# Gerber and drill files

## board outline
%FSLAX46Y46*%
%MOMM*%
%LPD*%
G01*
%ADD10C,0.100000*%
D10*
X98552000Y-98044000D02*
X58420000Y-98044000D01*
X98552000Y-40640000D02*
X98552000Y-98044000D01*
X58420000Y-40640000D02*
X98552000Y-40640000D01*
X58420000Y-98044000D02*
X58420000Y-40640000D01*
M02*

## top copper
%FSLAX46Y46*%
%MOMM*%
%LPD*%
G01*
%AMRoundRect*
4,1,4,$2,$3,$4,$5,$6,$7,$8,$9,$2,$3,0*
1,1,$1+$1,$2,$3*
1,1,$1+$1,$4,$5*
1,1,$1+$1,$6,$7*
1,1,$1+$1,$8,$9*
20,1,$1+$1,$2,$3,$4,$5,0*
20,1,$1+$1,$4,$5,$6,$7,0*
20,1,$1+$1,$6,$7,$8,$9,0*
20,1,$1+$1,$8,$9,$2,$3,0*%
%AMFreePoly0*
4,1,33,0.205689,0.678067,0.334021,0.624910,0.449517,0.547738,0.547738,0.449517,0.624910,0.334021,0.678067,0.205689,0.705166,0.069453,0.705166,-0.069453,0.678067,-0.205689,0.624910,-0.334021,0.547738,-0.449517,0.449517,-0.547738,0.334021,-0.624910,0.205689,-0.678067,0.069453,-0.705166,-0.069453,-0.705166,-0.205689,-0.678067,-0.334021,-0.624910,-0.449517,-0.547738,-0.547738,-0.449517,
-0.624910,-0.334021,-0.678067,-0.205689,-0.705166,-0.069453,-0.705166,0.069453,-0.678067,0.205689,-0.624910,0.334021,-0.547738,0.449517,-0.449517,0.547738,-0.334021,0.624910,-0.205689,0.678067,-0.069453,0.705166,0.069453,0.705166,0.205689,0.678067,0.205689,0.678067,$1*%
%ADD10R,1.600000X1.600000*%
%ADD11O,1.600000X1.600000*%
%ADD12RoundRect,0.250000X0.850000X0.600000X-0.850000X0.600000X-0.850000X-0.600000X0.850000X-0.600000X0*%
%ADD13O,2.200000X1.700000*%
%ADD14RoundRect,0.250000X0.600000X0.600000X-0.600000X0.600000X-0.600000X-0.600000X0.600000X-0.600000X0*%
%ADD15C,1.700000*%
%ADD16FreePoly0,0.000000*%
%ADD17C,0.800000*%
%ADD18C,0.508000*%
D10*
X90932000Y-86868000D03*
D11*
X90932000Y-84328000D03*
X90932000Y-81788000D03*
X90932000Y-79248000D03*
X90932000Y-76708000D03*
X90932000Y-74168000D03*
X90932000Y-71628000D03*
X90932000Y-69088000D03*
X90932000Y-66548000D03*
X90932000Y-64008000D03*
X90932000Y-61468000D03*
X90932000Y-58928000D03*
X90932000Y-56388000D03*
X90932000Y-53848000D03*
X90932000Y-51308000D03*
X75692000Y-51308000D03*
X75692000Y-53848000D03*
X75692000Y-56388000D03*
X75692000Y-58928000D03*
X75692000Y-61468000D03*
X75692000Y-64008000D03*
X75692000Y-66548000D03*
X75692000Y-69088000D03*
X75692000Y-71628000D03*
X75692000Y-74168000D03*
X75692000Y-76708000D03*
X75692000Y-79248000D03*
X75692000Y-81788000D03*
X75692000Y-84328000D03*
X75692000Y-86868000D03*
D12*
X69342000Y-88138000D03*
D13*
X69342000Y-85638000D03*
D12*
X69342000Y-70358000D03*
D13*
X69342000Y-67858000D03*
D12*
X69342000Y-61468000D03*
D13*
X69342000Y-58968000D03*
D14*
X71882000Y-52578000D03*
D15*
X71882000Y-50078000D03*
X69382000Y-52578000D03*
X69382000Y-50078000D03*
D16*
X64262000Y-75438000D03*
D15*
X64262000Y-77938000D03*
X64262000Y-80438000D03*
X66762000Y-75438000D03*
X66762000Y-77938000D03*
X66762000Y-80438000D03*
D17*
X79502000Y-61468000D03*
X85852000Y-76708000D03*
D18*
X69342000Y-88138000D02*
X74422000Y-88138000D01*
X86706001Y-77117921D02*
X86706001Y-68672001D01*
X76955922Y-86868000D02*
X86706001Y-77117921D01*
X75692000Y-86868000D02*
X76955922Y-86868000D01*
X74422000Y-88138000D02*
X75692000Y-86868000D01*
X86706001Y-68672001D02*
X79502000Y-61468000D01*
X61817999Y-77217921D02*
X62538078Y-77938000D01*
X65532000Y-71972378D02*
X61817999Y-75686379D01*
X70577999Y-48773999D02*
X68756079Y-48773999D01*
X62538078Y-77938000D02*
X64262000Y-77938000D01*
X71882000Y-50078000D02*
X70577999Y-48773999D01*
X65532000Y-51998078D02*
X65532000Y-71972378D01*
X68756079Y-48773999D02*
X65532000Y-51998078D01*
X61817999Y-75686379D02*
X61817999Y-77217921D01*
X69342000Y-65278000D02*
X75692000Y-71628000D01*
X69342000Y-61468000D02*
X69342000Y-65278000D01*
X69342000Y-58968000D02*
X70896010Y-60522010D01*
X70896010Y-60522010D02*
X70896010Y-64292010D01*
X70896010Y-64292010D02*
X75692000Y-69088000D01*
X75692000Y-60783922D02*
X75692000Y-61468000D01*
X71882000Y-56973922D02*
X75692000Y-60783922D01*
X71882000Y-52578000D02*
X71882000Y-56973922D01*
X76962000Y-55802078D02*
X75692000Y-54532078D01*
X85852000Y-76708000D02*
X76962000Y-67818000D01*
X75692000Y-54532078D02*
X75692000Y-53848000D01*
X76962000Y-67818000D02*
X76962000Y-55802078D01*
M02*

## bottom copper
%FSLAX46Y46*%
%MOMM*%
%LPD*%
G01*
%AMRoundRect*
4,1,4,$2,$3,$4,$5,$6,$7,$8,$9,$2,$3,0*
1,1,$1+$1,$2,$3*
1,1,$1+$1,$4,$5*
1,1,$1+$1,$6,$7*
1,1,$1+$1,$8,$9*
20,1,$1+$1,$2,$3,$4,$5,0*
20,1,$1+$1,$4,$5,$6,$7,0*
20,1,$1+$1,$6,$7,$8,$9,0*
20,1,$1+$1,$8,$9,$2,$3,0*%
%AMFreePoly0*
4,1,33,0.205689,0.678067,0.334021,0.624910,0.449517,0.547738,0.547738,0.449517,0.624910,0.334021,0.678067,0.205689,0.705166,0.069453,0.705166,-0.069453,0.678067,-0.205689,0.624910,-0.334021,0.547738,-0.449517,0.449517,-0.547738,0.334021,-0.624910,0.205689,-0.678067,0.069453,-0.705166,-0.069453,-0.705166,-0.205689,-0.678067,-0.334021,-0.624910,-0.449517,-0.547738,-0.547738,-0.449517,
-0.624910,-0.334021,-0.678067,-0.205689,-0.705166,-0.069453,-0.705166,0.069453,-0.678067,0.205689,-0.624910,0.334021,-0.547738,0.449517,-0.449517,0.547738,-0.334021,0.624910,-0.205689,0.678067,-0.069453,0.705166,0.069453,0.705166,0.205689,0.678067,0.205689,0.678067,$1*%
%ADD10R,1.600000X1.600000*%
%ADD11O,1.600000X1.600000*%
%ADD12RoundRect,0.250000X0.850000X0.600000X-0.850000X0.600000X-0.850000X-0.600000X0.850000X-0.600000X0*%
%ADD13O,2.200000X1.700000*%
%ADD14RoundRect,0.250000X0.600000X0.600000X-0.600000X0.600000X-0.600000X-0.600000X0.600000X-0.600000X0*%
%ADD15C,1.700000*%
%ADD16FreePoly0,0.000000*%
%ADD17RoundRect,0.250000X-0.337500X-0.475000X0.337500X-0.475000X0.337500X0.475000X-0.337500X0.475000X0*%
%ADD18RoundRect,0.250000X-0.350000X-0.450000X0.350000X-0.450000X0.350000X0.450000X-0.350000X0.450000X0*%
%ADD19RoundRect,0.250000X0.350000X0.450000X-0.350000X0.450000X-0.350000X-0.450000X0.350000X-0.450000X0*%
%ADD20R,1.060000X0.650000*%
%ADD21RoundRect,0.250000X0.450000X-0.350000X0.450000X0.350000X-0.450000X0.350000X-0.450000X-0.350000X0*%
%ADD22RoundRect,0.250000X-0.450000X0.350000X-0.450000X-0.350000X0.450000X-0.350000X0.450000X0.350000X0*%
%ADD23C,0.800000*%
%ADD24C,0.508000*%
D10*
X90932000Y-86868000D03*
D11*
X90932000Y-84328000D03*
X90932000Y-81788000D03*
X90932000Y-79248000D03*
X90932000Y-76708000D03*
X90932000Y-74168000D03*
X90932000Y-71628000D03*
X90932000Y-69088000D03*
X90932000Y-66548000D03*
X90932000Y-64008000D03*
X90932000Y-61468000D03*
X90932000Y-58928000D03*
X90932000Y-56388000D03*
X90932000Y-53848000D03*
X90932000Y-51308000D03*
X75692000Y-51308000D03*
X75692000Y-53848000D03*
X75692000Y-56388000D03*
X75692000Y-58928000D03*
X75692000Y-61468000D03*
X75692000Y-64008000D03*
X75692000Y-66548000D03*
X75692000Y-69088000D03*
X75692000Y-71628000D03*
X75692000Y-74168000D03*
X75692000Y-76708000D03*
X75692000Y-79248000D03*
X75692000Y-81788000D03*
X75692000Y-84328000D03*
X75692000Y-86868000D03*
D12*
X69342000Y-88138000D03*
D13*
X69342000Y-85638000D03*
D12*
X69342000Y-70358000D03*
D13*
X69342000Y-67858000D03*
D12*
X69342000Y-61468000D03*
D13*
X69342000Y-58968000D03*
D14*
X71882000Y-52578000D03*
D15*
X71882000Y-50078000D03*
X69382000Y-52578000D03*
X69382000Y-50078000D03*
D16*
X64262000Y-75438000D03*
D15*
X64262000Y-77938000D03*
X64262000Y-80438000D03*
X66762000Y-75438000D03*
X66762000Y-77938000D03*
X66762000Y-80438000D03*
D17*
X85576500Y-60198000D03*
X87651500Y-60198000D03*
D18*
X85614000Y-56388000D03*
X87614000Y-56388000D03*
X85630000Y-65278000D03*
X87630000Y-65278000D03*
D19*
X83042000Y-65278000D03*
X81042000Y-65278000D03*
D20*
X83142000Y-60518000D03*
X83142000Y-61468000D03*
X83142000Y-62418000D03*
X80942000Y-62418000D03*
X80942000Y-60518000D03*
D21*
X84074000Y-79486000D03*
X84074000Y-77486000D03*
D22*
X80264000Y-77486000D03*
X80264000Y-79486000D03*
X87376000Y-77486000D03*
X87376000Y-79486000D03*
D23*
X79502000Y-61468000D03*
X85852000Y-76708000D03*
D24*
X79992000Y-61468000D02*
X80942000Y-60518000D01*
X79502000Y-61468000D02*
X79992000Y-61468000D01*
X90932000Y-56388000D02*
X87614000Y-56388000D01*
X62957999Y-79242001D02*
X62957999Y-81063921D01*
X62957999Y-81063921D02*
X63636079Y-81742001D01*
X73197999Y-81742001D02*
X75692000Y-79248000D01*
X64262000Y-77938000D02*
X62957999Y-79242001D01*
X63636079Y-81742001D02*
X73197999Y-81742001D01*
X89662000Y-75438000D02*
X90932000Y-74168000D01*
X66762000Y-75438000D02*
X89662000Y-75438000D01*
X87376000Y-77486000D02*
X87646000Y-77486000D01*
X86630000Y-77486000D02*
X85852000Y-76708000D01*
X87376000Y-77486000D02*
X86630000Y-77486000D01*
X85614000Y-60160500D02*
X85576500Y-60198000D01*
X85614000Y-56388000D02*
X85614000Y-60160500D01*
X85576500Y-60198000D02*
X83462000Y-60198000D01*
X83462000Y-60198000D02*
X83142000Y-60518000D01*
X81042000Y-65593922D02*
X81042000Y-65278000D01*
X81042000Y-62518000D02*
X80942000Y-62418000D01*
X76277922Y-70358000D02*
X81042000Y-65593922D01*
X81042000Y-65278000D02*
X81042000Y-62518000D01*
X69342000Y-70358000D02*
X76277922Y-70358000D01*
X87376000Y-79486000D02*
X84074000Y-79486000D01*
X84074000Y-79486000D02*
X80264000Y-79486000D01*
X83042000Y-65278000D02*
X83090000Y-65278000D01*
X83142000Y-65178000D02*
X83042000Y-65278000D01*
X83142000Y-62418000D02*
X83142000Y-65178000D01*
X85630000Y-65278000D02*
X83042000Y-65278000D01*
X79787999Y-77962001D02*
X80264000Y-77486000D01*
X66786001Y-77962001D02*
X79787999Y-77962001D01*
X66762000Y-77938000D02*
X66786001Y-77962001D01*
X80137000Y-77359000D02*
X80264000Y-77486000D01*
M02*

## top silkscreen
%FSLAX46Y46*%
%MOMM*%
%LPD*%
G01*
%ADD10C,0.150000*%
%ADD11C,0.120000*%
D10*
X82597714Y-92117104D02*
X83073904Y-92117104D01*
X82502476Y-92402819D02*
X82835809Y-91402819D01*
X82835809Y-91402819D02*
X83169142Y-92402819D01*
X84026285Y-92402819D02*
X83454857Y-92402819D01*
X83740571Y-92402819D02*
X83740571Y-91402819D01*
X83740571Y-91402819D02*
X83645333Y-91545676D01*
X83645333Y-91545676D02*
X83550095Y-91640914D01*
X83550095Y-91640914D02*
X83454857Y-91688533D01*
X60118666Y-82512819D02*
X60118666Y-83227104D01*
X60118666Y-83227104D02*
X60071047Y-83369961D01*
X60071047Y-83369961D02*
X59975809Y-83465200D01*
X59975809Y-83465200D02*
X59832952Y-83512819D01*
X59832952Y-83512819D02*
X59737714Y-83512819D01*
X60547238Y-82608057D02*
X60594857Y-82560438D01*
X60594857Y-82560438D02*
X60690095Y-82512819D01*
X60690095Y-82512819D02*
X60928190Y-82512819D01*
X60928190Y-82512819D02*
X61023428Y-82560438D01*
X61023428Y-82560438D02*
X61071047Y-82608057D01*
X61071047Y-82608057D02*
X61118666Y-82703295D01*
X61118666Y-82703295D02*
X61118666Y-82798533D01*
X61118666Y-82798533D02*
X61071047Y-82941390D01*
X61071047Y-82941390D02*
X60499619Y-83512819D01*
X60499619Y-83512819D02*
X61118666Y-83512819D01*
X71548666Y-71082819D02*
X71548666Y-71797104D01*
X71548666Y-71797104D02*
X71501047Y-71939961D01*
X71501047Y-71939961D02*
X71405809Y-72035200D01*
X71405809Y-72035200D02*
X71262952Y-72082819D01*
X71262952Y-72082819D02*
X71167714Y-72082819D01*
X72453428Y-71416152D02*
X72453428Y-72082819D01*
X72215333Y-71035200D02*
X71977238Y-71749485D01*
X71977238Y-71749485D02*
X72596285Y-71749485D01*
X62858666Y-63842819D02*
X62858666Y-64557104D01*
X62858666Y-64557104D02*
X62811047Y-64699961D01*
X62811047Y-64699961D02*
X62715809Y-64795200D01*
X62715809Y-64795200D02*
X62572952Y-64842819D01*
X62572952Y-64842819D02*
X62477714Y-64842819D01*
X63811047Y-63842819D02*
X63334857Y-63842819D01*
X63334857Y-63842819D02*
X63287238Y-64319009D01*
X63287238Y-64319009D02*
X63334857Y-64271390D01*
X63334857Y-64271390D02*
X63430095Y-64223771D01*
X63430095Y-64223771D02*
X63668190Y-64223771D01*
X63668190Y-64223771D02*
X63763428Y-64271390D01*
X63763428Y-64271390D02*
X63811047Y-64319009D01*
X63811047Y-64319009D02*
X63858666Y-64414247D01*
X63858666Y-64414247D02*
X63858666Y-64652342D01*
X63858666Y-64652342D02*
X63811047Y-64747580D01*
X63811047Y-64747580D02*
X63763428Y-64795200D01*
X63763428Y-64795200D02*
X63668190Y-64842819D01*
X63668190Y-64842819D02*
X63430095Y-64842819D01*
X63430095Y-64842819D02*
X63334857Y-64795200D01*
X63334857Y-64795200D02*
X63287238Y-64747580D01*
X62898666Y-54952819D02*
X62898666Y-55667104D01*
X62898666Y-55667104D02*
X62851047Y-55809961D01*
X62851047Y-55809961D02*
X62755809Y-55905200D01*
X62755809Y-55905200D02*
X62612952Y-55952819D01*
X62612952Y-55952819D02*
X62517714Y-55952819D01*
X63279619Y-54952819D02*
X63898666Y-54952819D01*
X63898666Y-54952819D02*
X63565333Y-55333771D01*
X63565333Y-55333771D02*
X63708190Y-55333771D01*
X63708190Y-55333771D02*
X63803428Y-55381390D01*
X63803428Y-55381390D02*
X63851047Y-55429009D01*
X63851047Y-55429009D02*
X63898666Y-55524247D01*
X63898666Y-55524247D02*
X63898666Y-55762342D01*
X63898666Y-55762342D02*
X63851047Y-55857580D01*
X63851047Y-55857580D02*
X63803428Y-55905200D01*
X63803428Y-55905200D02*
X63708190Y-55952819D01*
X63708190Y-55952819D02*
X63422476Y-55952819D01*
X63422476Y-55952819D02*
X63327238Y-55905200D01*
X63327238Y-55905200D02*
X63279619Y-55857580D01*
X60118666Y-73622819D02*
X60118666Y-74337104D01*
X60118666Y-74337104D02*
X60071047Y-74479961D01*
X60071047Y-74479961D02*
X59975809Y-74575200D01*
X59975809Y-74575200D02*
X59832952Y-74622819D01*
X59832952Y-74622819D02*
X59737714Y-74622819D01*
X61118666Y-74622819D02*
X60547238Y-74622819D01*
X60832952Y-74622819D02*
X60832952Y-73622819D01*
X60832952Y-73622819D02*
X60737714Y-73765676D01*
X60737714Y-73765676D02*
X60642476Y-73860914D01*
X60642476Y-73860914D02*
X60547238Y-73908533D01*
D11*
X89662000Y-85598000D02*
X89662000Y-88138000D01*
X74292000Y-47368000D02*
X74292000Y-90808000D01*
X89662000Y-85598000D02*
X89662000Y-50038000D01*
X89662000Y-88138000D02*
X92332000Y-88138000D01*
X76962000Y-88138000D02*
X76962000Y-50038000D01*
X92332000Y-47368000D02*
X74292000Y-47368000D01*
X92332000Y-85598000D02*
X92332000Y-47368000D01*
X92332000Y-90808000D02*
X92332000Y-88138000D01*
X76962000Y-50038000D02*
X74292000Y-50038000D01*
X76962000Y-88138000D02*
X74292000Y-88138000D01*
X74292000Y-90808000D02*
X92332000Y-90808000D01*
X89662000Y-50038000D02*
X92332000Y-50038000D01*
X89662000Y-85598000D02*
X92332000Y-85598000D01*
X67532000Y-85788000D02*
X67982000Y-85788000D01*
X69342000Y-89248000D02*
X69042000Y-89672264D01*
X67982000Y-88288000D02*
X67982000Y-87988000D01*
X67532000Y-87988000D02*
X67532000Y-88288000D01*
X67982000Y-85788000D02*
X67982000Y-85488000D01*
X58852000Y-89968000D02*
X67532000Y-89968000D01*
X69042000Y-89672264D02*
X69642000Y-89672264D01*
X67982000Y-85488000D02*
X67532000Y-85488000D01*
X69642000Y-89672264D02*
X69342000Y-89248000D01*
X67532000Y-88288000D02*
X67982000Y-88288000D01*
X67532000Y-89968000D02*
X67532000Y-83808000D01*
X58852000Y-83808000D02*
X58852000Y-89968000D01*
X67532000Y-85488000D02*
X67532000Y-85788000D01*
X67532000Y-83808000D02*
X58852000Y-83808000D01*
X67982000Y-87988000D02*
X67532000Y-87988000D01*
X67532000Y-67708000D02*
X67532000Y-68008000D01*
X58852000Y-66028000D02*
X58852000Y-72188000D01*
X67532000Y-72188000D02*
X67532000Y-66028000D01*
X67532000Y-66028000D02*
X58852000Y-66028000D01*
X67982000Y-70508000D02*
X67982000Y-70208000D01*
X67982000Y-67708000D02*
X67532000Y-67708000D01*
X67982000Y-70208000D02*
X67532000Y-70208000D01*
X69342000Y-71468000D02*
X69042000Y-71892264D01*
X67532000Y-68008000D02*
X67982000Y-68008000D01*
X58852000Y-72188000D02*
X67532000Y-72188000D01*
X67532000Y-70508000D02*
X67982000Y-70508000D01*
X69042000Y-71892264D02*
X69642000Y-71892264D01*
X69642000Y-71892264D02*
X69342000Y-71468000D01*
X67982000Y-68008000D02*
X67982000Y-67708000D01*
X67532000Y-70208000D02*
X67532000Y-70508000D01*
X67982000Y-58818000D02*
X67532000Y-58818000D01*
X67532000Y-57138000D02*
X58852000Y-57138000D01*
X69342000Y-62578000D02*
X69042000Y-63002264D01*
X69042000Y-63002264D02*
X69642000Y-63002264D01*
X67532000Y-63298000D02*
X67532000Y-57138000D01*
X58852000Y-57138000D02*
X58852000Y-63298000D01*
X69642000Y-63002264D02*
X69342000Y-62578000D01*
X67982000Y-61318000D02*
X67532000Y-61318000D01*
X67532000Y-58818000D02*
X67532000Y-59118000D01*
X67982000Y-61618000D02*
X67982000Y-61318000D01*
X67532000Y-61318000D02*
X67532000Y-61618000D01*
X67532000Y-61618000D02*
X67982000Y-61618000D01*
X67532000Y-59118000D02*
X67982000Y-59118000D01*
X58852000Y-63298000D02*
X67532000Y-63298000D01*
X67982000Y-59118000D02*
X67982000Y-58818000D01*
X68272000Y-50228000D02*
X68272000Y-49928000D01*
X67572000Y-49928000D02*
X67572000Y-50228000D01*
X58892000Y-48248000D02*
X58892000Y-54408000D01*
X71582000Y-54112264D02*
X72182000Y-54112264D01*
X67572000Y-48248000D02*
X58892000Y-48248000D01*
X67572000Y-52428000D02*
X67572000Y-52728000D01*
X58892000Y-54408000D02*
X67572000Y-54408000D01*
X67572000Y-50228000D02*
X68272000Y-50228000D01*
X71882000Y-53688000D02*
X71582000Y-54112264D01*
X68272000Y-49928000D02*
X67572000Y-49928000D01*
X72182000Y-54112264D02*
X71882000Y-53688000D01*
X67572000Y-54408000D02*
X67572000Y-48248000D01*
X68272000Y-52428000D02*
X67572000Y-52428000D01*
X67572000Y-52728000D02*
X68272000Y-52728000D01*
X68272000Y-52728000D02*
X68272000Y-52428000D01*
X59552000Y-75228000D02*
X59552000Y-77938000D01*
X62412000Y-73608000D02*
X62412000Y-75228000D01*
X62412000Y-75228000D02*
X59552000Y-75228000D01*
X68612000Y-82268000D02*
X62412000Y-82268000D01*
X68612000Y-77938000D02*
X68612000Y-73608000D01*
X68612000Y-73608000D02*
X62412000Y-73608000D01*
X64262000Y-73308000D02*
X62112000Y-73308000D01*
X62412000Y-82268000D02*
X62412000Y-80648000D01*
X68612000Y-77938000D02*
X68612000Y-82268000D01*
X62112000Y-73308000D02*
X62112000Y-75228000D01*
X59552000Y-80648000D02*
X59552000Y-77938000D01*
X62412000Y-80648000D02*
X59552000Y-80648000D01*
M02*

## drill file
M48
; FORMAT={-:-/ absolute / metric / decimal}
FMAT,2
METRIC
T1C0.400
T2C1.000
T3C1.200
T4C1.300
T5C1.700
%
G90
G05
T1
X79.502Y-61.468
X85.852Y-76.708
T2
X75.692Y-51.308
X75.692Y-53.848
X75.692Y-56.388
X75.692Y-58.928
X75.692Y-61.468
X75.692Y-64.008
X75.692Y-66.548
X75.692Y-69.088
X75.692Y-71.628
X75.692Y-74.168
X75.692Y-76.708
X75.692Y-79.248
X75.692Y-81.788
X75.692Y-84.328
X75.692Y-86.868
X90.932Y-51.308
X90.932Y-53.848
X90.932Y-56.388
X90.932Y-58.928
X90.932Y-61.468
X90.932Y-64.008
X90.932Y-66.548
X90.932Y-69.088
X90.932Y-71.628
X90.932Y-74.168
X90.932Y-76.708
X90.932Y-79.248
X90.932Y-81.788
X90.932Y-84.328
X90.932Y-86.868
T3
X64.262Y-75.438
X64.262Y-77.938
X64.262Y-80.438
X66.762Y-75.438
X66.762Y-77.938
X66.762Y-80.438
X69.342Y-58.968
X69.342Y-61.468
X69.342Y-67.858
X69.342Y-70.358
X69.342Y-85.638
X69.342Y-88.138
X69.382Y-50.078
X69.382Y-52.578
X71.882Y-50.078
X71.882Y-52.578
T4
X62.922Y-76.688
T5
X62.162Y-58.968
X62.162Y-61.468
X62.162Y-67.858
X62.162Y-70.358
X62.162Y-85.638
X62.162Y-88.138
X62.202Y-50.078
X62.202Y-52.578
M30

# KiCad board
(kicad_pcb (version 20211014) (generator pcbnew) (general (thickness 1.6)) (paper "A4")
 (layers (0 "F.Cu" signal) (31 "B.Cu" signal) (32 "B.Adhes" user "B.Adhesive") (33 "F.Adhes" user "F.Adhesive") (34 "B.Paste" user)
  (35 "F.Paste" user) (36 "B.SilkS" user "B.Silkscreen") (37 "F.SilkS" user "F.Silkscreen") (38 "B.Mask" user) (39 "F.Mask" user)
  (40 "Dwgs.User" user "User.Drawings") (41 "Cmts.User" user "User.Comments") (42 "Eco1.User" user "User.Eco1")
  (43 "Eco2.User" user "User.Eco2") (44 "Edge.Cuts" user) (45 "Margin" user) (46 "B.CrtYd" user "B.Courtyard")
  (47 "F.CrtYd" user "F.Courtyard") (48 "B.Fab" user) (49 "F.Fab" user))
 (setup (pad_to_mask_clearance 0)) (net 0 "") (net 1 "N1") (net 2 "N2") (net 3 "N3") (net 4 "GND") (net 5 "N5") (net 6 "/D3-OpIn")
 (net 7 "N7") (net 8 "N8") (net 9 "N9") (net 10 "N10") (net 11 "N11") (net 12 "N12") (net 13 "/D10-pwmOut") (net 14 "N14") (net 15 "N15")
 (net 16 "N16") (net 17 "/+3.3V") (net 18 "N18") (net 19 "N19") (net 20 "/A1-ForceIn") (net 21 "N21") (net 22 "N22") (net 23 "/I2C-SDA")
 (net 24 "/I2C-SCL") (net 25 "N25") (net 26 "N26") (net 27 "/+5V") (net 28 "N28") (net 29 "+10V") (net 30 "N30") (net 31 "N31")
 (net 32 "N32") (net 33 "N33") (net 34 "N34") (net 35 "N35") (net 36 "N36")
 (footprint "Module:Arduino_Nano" (layer "F.Cu") (at 90.932 86.868 180)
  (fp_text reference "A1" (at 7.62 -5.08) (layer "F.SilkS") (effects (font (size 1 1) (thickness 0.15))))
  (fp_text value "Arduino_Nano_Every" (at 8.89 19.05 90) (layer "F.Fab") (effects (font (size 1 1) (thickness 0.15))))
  (fp_line (start 1.27 1.27) (end 1.27 -1.27) (layer "F.SilkS") (width 0.12))
  (fp_line (start 16.64 39.5) (end 16.64 -3.94) (layer "F.SilkS") (width 0.12))
  (fp_line (start 1.27 1.27) (end 1.27 36.83) (layer "F.SilkS") (width 0.12))
  (fp_line (start 1.27 -1.27) (end -1.4 -1.27) (layer "F.SilkS") (width 0.12))
  (fp_line (start 13.97 -1.27) (end 13.97 36.83) (layer "F.SilkS") (width 0.12))
  (fp_line (start -1.4 39.5) (end 16.64 39.5) (layer "F.SilkS") (width 0.12))
  (fp_line (start -1.4 1.27) (end -1.4 39.5) (layer "F.SilkS") (width 0.12))
  (fp_line (start -1.4 -3.94) (end -1.4 -1.27) (layer "F.SilkS") (width 0.12))
  (fp_line (start 13.97 36.83) (end 16.64 36.83) (layer "F.SilkS") (width 0.12))
  (fp_line (start 13.97 -1.27) (end 16.64 -1.27) (layer "F.SilkS") (width 0.12))
  (fp_line (start 16.64 -3.94) (end -1.4 -3.94) (layer "F.SilkS") (width 0.12))
  (fp_line (start 1.27 36.83) (end -1.4 36.83) (layer "F.SilkS") (width 0.12))
  (fp_line (start 1.27 1.27) (end -1.4 1.27) (layer "F.SilkS") (width 0.12))
  (pad "1" thru_hole rect locked (at 0 0 180) (size 1.6 1.6) (drill 1) (layers *.Cu *.Mask) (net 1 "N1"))
  (pad "2" thru_hole oval locked (at 0 2.54 180) (size 1.6 1.6) (drill 1) (layers *.Cu *.Mask) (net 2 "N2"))
  (pad "3" thru_hole oval locked (at 0 5.08 180) (size 1.6 1.6) (drill 1) (layers *.Cu *.Mask) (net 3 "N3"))
  (pad "4" thru_hole oval locked (at 0 7.62 180) (size 1.6 1.6) (drill 1) (layers *.Cu *.Mask) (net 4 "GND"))
  (pad "5" thru_hole oval locked (at 0 10.16 180) (size 1.6 1.6) (drill 1) (layers *.Cu *.Mask) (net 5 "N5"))
  (pad "6" thru_hole oval locked (at 0 12.7 180) (size 1.6 1.6) (drill 1) (layers *.Cu *.Mask) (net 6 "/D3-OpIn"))
  (pad "7" thru_hole oval locked (at 0 15.24 180) (size 1.6 1.6) (drill 1) (layers *.Cu *.Mask) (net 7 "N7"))
  (pad "8" thru_hole oval locked (at 0 17.78 180) (size 1.6 1.6) (drill 1) (layers *.Cu *.Mask) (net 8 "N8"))
  (pad "9" thru_hole oval locked (at 0 20.32 180) (size 1.6 1.6) (drill 1) (layers *.Cu *.Mask) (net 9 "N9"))
  (pad "10" thru_hole oval locked (at 0 22.86 180) (size 1.6 1.6) (drill 1) (layers *.Cu *.Mask) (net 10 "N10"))
  (pad "11" thru_hole oval locked (at 0 25.4 180) (size 1.6 1.6) (drill 1) (layers *.Cu *.Mask) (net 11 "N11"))
  (pad "12" thru_hole oval locked (at 0 27.94 180) (size 1.6 1.6) (drill 1) (layers *.Cu *.Mask) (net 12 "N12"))
  (pad "13" thru_hole oval locked (at 0 30.48 180) (size 1.6 1.6) (drill 1) (layers *.Cu *.Mask) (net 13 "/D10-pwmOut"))
  (pad "14" thru_hole oval locked (at 0 33.02 180) (size 1.6 1.6) (drill 1) (layers *.Cu *.Mask) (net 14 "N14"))
  (pad "15" thru_hole oval locked (at 0 35.56 180) (size 1.6 1.6) (drill 1) (layers *.Cu *.Mask) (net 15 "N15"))
  (pad "16" thru_hole oval locked (at 15.24 35.56 180) (size 1.6 1.6) (drill 1) (layers *.Cu *.Mask) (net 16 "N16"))
  (pad "17" thru_hole oval locked (at 15.24 33.02 180) (size 1.6 1.6) (drill 1) (layers *.Cu *.Mask) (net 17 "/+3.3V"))
  (pad "18" thru_hole oval locked (at 15.24 30.48 180) (size 1.6 1.6) (drill 1) (layers *.Cu *.Mask) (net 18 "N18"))
  (pad "19" thru_hole oval locked (at 15.24 27.94 180) (size 1.6 1.6) (drill 1) (layers *.Cu *.Mask) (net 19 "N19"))
  (pad "20" thru_hole oval locked (at 15.24 25.4 180) (size 1.6 1.6) (drill 1) (layers *.Cu *.Mask) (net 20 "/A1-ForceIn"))
  (pad "21" thru_hole oval locked (at 15.24 22.86 180) (size 1.6 1.6) (drill 1) (layers *.Cu *.Mask) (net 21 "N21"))
  (pad "22" thru_hole oval locked (at 15.24 20.32 180) (size 1.6 1.6) (drill 1) (layers *.Cu *.Mask) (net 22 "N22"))
  (pad "23" thru_hole oval locked (at 15.24 17.78 180) (size 1.6 1.6) (drill 1) (layers *.Cu *.Mask) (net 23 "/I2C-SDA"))
  (pad "24" thru_hole oval locked (at 15.24 15.24 180) (size 1.6 1.6) (drill 1) (layers *.Cu *.Mask) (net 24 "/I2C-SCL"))
  (pad "25" thru_hole oval locked (at 15.24 12.7 180) (size 1.6 1.6) (drill 1) (layers *.Cu *.Mask) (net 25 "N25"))
  (pad "26" thru_hole oval locked (at 15.24 10.16 180) (size 1.6 1.6) (drill 1) (layers *.Cu *.Mask) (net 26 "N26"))
  (pad "27" thru_hole oval locked (at 15.24 7.62 180) (size 1.6 1.6) (drill 1) (layers *.Cu *.Mask) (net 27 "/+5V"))
  (pad "28" thru_hole oval locked (at 15.24 5.08 180) (size 1.6 1.6) (drill 1) (layers *.Cu *.Mask) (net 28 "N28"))
  (pad "29" thru_hole oval locked (at 15.24 2.54 180) (size 1.6 1.6) (drill 1) (layers *.Cu *.Mask) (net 4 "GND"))
  (pad "30" thru_hole oval locked (at 15.24 0 180) (size 1.6 1.6) (drill 1) (layers *.Cu *.Mask) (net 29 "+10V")))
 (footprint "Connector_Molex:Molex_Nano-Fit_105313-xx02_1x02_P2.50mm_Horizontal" (layer "F.Cu") (at 69.342 88.138 180)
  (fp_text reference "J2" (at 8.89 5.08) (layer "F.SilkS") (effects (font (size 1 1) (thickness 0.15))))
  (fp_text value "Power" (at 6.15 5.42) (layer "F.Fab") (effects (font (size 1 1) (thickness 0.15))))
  (fp_line (start 1.81 2.35) (end 1.36 2.35) (layer "F.SilkS") (width 0.12))
  (fp_line (start 0 -1.11) (end 0.3 -1.534264) (layer "F.SilkS") (width 0.12))
  (fp_line (start 1.36 -0.15) (end 1.36 0.15) (layer "F.SilkS") (width 0.12))
  (fp_line (start 1.81 0.15) (end 1.81 -0.15) (layer "F.SilkS") (width 0.12))
  (fp_line (start 1.36 2.35) (end 1.36 2.65) (layer "F.SilkS") (width 0.12))
  (fp_line (start 10.49 -1.83) (end 1.81 -1.83) (layer "F.SilkS") (width 0.12))
  (fp_line (start 0.3 -1.534264) (end -0.3 -1.534264) (layer "F.SilkS") (width 0.12))
  (fp_line (start 1.36 2.65) (end 1.81 2.65) (layer "F.SilkS") (width 0.12))
  (fp_line (start -0.3 -1.534264) (end 0 -1.11) (layer "F.SilkS") (width 0.12))
  (fp_line (start 1.81 -0.15) (end 1.36 -0.15) (layer "F.SilkS") (width 0.12))
  (fp_line (start 1.81 -1.83) (end 1.81 4.33) (layer "F.SilkS") (width 0.12))
  (fp_line (start 10.49 4.33) (end 10.49 -1.83) (layer "F.SilkS") (width 0.12))
  (fp_line (start 1.81 2.65) (end 1.81 2.35) (layer "F.SilkS") (width 0.12))
  (fp_line (start 1.81 4.33) (end 10.49 4.33) (layer "F.SilkS") (width 0.12))
  (fp_line (start 1.36 0.15) (end 1.81 0.15) (layer "F.SilkS") (width 0.12))
  (pad "" np_thru_hole circle locked (at 7.18 2.5 180) (size 1.7 1.7) (drill 1.7) (layers *.Cu *.Mask))
  (pad "" np_thru_hole circle locked (at 7.18 0 180) (size 1.7 1.7) (drill 1.7) (layers *.Cu *.Mask))
  (pad "1" thru_hole roundrect locked (at 0 0 180) (size 2.2 1.7) (drill 1.2) (layers *.Cu *.Mask) (roundrect_rratio 0.147059)
   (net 29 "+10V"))
  (pad "2" thru_hole oval locked (at 0 2.5 180) (size 2.2 1.7) (drill 1.2) (layers *.Cu *.Mask) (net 4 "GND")))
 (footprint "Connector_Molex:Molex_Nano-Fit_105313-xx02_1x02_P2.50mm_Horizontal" (layer "F.Cu") (at 69.342 70.358 180)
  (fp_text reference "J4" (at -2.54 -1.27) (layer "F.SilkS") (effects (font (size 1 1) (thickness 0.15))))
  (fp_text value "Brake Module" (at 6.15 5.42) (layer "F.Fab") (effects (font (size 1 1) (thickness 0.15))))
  (fp_line (start 1.81 2.65) (end 1.81 2.35) (layer "F.SilkS") (width 0.12))
  (fp_line (start 10.49 4.33) (end 10.49 -1.83) (layer "F.SilkS") (width 0.12))
  (fp_line (start 1.81 -1.83) (end 1.81 4.33) (layer "F.SilkS") (width 0.12))
  (fp_line (start 1.81 4.33) (end 10.49 4.33) (layer "F.SilkS") (width 0.12))
  (fp_line (start 1.36 -0.15) (end 1.36 0.15) (layer "F.SilkS") (width 0.12))
  (fp_line (start 1.36 2.65) (end 1.81 2.65) (layer "F.SilkS") (width 0.12))
  (fp_line (start 1.36 0.15) (end 1.81 0.15) (layer "F.SilkS") (width 0.12))
  (fp_line (start 0 -1.11) (end 0.3 -1.534264) (layer "F.SilkS") (width 0.12))
  (fp_line (start 1.81 2.35) (end 1.36 2.35) (layer "F.SilkS") (width 0.12))
  (fp_line (start 10.49 -1.83) (end 1.81 -1.83) (layer "F.SilkS") (width 0.12))
  (fp_line (start 1.81 -0.15) (end 1.36 -0.15) (layer "F.SilkS") (width 0.12))
  (fp_line (start 0.3 -1.534264) (end -0.3 -1.534264) (layer "F.SilkS") (width 0.12))
  (fp_line (start -0.3 -1.534264) (end 0 -1.11) (layer "F.SilkS") (width 0.12))
  (fp_line (start 1.36 2.35) (end 1.36 2.65) (layer "F.SilkS") (width 0.12))
  (fp_line (start 1.81 0.15) (end 1.81 -0.15) (layer "F.SilkS") (width 0.12))
  (pad "" np_thru_hole circle locked (at 7.18 0 180) (size 1.7 1.7) (drill 1.7) (layers *.Cu *.Mask))
  (pad "" np_thru_hole circle locked (at 7.18 2.5 180) (size 1.7 1.7) (drill 1.7) (layers *.Cu *.Mask))
  (pad "1" thru_hole roundrect locked (at 0 0 180) (size 2.2 1.7) (drill 1.2) (layers *.Cu *.Mask) (roundrect_rratio 0.147059)
   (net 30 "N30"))
  (pad "2" thru_hole oval locked (at 0 2.5 180) (size 2.2 1.7) (drill 1.2) (layers *.Cu *.Mask) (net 4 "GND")))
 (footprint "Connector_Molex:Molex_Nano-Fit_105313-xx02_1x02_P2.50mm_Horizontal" (layer "F.Cu") (at 69.342 61.468 180)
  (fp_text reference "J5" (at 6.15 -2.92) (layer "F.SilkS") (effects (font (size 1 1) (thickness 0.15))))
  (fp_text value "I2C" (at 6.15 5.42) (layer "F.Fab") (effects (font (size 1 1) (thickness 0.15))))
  (fp_line (start 1.36 2.65) (end 1.81 2.65) (layer "F.SilkS") (width 0.12))
  (fp_line (start 1.81 4.33) (end 10.49 4.33) (layer "F.SilkS") (width 0.12))
  (fp_line (start 0 -1.11) (end 0.3 -1.534264) (layer "F.SilkS") (width 0.12))
  (fp_line (start 0.3 -1.534264) (end -0.3 -1.534264) (layer "F.SilkS") (width 0.12))
  (fp_line (start 1.81 -1.83) (end 1.81 4.33) (layer "F.SilkS") (width 0.12))
  (fp_line (start 10.49 4.33) (end 10.49 -1.83) (layer "F.SilkS") (width 0.12))
  (fp_line (start -0.3 -1.534264) (end 0 -1.11) (layer "F.SilkS") (width 0.12))
  (fp_line (start 1.36 0.15) (end 1.81 0.15) (layer "F.SilkS") (width 0.12))
  (fp_line (start 1.81 2.65) (end 1.81 2.35) (layer "F.SilkS") (width 0.12))
  (fp_line (start 1.36 -0.15) (end 1.36 0.15) (layer "F.SilkS") (width 0.12))
  (fp_line (start 1.81 0.15) (end 1.81 -0.15) (layer "F.SilkS") (width 0.12))
  (fp_line (start 1.81 -0.15) (end 1.36 -0.15) (layer "F.SilkS") (width 0.12))
  (fp_line (start 1.81 2.35) (end 1.36 2.35) (layer "F.SilkS") (width 0.12))
  (fp_line (start 10.49 -1.83) (end 1.81 -1.83) (layer "F.SilkS") (width 0.12))
  (fp_line (start 1.36 2.35) (end 1.36 2.65) (layer "F.SilkS") (width 0.12))
  (pad "" np_thru_hole circle locked (at 7.18 0 180) (size 1.7 1.7) (drill 1.7) (layers *.Cu *.Mask))
  (pad "" np_thru_hole circle locked (at 7.18 2.5 180) (size 1.7 1.7) (drill 1.7) (layers *.Cu *.Mask))
  (pad "1" thru_hole roundrect locked (at 0 0 180) (size 2.2 1.7) (drill 1.2) (layers *.Cu *.Mask) (roundrect_rratio 0.147059)
   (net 24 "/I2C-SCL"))
  (pad "2" thru_hole oval locked (at 0 2.5 180) (size 2.2 1.7) (drill 1.2) (layers *.Cu *.Mask) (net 23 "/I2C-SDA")))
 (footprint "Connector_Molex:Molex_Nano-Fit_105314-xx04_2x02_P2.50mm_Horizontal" (layer "F.Cu") (at 71.882 52.578 180)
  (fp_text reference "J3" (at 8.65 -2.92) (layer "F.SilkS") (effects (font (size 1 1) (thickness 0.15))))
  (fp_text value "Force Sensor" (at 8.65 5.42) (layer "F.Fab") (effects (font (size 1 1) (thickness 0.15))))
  (fp_line (start 3.61 2.35) (end 3.61 2.65) (layer "F.SilkS") (width 0.12))
  (fp_line (start 4.31 2.65) (end 4.31 2.35) (layer "F.SilkS") (width 0.12))
  (fp_line (start 12.99 4.33) (end 12.99 -1.83) (layer "F.SilkS") (width 0.12))
  (fp_line (start 0.3 -1.534264) (end -0.3 -1.534264) (layer "F.SilkS") (width 0.12))
  (fp_line (start 4.31 4.33) (end 12.99 4.33) (layer "F.SilkS") (width 0.12))
  (fp_line (start 4.31 0.15) (end 4.31 -0.15) (layer "F.SilkS") (width 0.12))
  (fp_line (start 12.99 -1.83) (end 4.31 -1.83) (layer "F.SilkS") (width 0.12))
  (fp_line (start 4.31 2.35) (end 3.61 2.35) (layer "F.SilkS") (width 0.12))
  (fp_line (start 0 -1.11) (end 0.3 -1.534264) (layer "F.SilkS") (width 0.12))
  (fp_line (start 3.61 2.65) (end 4.31 2.65) (layer "F.SilkS") (width 0.12))
  (fp_line (start -0.3 -1.534264) (end 0 -1.11) (layer "F.SilkS") (width 0.12))
  (fp_line (start 4.31 -1.83) (end 4.31 4.33) (layer "F.SilkS") (width 0.12))
  (fp_line (start 3.61 0.15) (end 4.31 0.15) (layer "F.SilkS") (width 0.12))
  (fp_line (start 4.31 -0.15) (end 3.61 -0.15) (layer "F.SilkS") (width 0.12))
  (fp_line (start 3.61 -0.15) (end 3.61 0.15) (layer "F.SilkS") (width 0.12))
  (pad "" np_thru_hole circle locked (at 9.68 2.5 180) (size 1.7 1.7) (drill 1.7) (layers *.Cu *.Mask))
  (pad "" np_thru_hole circle locked (at 9.68 0 180) (size 1.7 1.7) (drill 1.7) (layers *.Cu *.Mask))
  (pad "1" thru_hole roundrect locked (at 0 0 180) (size 1.7 1.7) (drill 1.2) (layers *.Cu *.Mask) (roundrect_rratio 0.147059)
   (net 20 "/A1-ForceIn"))
  (pad "2" thru_hole circle locked (at 0 2.5 180) (size 1.7 1.7) (drill 1.2) (layers *.Cu *.Mask) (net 27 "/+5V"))
  (pad "3" thru_hole circle locked (at 2.5 0 180) (size 1.7 1.7) (drill 1.2) (layers *.Cu *.Mask) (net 4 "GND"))
  (pad "4" thru_hole circle locked (at 2.5 2.5 180) (size 1.7 1.7) (drill 1.2) (layers *.Cu *.Mask) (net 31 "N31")))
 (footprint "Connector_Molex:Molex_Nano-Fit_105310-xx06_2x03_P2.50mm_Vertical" (layer "F.Cu") (at 64.262 75.438)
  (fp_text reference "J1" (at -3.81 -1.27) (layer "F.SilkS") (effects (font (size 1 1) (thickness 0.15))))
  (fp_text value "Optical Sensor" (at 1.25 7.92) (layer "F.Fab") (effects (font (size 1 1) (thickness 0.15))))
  (fp_line (start -4.71 -0.21) (end -4.71 2.5) (layer "F.SilkS") (width 0.12))
  (fp_line (start -1.85 -1.83) (end -1.85 -0.21) (layer "F.SilkS") (width 0.12))
  (fp_line (start -1.85 -0.21) (end -4.71 -0.21) (layer "F.SilkS") (width 0.12))
  (fp_line (start 4.35 6.83) (end -1.85 6.83) (layer "F.SilkS") (width 0.12))
  (fp_line (start 4.35 2.5) (end 4.35 -1.83) (layer "F.SilkS") (width 0.12))
  (fp_line (start 4.35 -1.83) (end -1.85 -1.83) (layer "F.SilkS") (width 0.12))
  (fp_line (start 0 -2.13) (end -2.15 -2.13) (layer "F.SilkS") (width 0.12))
  (fp_line (start -1.85 6.83) (end -1.85 5.21) (layer "F.SilkS") (width 0.12))
  (fp_line (start 4.35 2.5) (end 4.35 6.83) (layer "F.SilkS") (width 0.12))
  (fp_line (start -2.15 -2.13) (end -2.15 -0.21) (layer "F.SilkS") (width 0.12))
  (fp_line (start -4.71 5.21) (end -4.71 2.5) (layer "F.SilkS") (width 0.12))
  (fp_line (start -1.85 5.21) (end -4.71 5.21) (layer "F.SilkS") (width 0.12))
  (pad "" np_thru_hole circle locked (at -1.34 1.25) (size 1.3 1.3) (drill 1.3) (layers *.Cu *.Mask))
  (pad "1" thru_hole custom locked (at 0 0) (size 1.417157 1.417157) (drill 1.2) (layers *.Cu *.Mask) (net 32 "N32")
   (options (clearance outline) (anchor circle)) (primitives))
  (pad "2" thru_hole circle locked (at 0 2.5) (size 1.7 1.7) (drill 1.2) (layers *.Cu *.Mask) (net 27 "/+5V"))
  (pad "3" thru_hole circle locked (at 0 5) (size 1.7 1.7) (drill 1.2) (layers *.Cu *.Mask) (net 4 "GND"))
  (pad "4" thru_hole circle locked (at 2.5 0) (size 1.7 1.7) (drill 1.2) (layers *.Cu *.Mask) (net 6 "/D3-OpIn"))
  (pad "5" thru_hole circle locked (at 2.5 2.5) (size 1.7 1.7) (drill 1.2) (layers *.Cu *.Mask) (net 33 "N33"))
  (pad "6" thru_hole circle locked (at 2.5 5) (size 1.7 1.7) (drill 1.2) (layers *.Cu *.Mask) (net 4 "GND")))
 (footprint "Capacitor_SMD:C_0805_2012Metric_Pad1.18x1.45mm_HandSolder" (layer "B.Cu") (at 86.614 60.198)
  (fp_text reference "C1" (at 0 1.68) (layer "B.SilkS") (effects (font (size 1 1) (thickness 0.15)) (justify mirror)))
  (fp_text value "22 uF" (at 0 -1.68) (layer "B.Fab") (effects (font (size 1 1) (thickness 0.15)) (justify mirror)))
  (pad "1" smd roundrect locked (at -1.0375 0) (size 1.175 1.45) (layers "B.Cu" "B.Paste" "B.Mask") (roundrect_rratio 0.212766)
   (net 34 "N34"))
  (pad "2" smd roundrect locked (at 1.0375 0) (size 1.175 1.45) (layers "B.Cu" "B.Paste" "B.Mask") (roundrect_rratio 0.212766) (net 4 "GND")))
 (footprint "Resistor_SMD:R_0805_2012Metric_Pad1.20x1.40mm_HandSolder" (layer "B.Cu") (at 86.614 56.388)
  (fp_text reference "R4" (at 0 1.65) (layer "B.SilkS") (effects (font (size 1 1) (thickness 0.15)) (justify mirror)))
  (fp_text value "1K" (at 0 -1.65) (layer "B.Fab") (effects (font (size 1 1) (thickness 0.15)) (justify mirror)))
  (pad "1" smd roundrect locked (at -1 0) (size 1.2 1.4) (layers "B.Cu" "B.Paste" "B.Mask") (roundrect_rratio 0.208333) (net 34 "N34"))
  (pad "2" smd roundrect locked (at 1 0) (size 1.2 1.4) (layers "B.Cu" "B.Paste" "B.Mask") (roundrect_rratio 0.208333)
   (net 13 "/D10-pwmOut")))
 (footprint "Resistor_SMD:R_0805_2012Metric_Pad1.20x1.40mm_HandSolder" (layer "B.Cu") (at 86.63 65.278)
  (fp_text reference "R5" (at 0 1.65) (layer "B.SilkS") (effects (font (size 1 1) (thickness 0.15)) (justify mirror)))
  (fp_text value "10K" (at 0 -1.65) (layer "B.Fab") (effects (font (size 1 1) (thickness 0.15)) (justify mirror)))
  (pad "1" smd roundrect locked (at -1 0) (size 1.2 1.4) (layers "B.Cu" "B.Paste" "B.Mask") (roundrect_rratio 0.208333) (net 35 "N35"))
  (pad "2" smd roundrect locked (at 1 0) (size 1.2 1.4) (layers "B.Cu" "B.Paste" "B.Mask") (roundrect_rratio 0.208333) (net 4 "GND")))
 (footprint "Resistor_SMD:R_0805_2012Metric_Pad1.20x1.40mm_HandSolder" (layer "B.Cu") (at 82.042 65.278 180)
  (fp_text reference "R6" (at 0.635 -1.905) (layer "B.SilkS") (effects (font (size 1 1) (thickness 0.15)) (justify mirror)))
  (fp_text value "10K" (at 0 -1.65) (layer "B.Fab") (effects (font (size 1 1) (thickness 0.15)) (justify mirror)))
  (pad "1" smd roundrect locked (at -1 0 180) (size 1.2 1.4) (layers "B.Cu" "B.Paste" "B.Mask") (roundrect_rratio 0.208333) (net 35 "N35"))
  (pad "2" smd roundrect locked (at 1 0 180) (size 1.2 1.4) (layers "B.Cu" "B.Paste" "B.Mask") (roundrect_rratio 0.208333) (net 30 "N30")))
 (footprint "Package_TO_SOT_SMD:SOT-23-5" (layer "B.Cu") (at 82.042 61.468 180)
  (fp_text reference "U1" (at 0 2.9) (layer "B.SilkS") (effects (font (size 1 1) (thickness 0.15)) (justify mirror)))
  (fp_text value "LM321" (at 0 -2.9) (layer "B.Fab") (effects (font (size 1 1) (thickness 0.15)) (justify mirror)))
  (pad "1" smd rect locked (at -1.1 0.95 180) (size 1.06 0.65) (layers "B.Cu" "B.Paste" "B.Mask") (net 34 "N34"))
  (pad "2" smd rect locked (at -1.1 0 180) (size 1.06 0.65) (layers "B.Cu" "B.Paste" "B.Mask") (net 4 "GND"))
  (pad "3" smd rect locked (at -1.1 -0.95 180) (size 1.06 0.65) (layers "B.Cu" "B.Paste" "B.Mask") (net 35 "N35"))
  (pad "4" smd rect locked (at 1.1 -0.95 180) (size 1.06 0.65) (layers "B.Cu" "B.Paste" "B.Mask") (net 30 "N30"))
  (pad "5" smd rect locked (at 1.1 0.95 180) (size 1.06 0.65) (layers "B.Cu" "B.Paste" "B.Mask") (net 29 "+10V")))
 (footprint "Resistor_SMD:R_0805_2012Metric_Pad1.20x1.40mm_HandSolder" (layer "B.Cu") (at 84.074 78.486 90)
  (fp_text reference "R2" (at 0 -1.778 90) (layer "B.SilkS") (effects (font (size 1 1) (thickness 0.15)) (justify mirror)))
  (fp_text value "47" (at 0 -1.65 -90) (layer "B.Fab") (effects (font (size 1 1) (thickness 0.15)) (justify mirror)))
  (pad "1" smd roundrect locked (at -1 0 90) (size 1.2 1.4) (layers "B.Cu" "B.Paste" "B.Mask") (roundrect_rratio 0.208333) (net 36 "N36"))
  (pad "2" smd roundrect locked (at 1 0 90) (size 1.2 1.4) (layers "B.Cu" "B.Paste" "B.Mask") (roundrect_rratio 0.208333) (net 4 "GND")))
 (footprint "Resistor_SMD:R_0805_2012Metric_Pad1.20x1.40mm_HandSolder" (layer "B.Cu") (at 80.264 78.486 -90)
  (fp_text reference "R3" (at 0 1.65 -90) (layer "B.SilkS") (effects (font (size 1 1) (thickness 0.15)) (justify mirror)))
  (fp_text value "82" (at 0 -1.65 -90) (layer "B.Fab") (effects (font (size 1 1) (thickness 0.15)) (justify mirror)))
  (pad "1" smd roundrect locked (at -1 0 270) (size 1.2 1.4) (layers "B.Cu" "B.Paste" "B.Mask") (roundrect_rratio 0.208333) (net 33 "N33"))
  (pad "2" smd roundrect locked (at 1 0 270) (size 1.2 1.4) (layers "B.Cu" "B.Paste" "B.Mask") (roundrect_rratio 0.208333) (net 36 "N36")))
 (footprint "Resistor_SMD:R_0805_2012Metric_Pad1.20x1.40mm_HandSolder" (layer "B.Cu") (at 87.376 78.486 -90)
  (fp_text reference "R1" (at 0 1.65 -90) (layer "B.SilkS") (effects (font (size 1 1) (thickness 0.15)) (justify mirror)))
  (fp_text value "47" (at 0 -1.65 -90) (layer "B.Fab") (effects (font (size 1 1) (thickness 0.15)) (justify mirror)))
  (pad "1" smd roundrect locked (at -1 0 270) (size 1.2 1.4) (layers "B.Cu" "B.Paste" "B.Mask") (roundrect_rratio 0.208333)
   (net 17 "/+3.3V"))
  (pad "2" smd roundrect locked (at 1 0 270) (size 1.2 1.4) (layers "B.Cu" "B.Paste" "B.Mask") (roundrect_rratio 0.208333) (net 36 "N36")))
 (gr_line (start 98.552 98.044) (end 58.42 98.044) (layer "Edge.Cuts") (width 0.1))
 (gr_line (start 98.552 40.64) (end 98.552 98.044) (layer "Edge.Cuts") (width 0.1))
 (gr_line (start 58.42 40.64) (end 98.552 40.64) (layer "Edge.Cuts") (width 0.1))
 (gr_line (start 58.42 98.044) (end 58.42 40.64) (layer "Edge.Cuts") (width 0.1))
 (segment (start 69.342 88.138) (end 74.422 88.138) (width 0.508) (layer "F.Cu") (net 29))
 (segment (start 86.706001 77.117921) (end 86.706001 68.672001) (width 0.508) (layer "F.Cu") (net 29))
 (segment (start 76.955922 86.868) (end 86.706001 77.117921) (width 0.508) (layer "F.Cu") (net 29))
 (segment (start 75.692 86.868) (end 76.955922 86.868) (width 0.508) (layer "F.Cu") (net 29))
 (segment (start 74.422 88.138) (end 75.692 86.868) (width 0.508) (layer "F.Cu") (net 29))
 (segment (start 86.706001 68.672001) (end 79.502 61.468) (width 0.508) (layer "F.Cu") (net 29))
 (via (at 79.502 61.468) (size 0.8) (drill 0.4) (layers "F.Cu" "B.Cu") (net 29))
 (segment (start 79.992 61.468) (end 80.942 60.518) (width 0.508) (layer "B.Cu") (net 29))
 (segment (start 79.502 61.468) (end 79.992 61.468) (width 0.508) (layer "B.Cu") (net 29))
 (segment (start 90.932 56.388) (end 87.614 56.388) (width 0.508) (layer "B.Cu") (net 13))
 (segment (start 61.817999 77.217921) (end 62.538078 77.938) (width 0.508) (layer "F.Cu") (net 27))
 (segment (start 65.532 71.972378) (end 61.817999 75.686379) (width 0.508) (layer "F.Cu") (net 27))
 (segment (start 70.577999 48.773999) (end 68.756079 48.773999) (width 0.508) (layer "F.Cu") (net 27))
 (segment (start 62.538078 77.938) (end 64.262 77.938) (width 0.508) (layer "F.Cu") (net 27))
 (segment (start 71.882 50.078) (end 70.577999 48.773999) (width 0.508) (layer "F.Cu") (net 27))
 (segment (start 65.532 51.998078) (end 65.532 71.972378) (width 0.508) (layer "F.Cu") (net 27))
 (segment (start 68.756079 48.773999) (end 65.532 51.998078) (width 0.508) (layer "F.Cu") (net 27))
 (segment (start 61.817999 75.686379) (end 61.817999 77.217921) (width 0.508) (layer "F.Cu") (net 27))
 (segment (start 62.957999 79.242001) (end 62.957999 81.063921) (width 0.508) (layer "B.Cu") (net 27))
 (segment (start 62.957999 81.063921) (end 63.636079 81.742001) (width 0.508) (layer "B.Cu") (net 27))
 (segment (start 73.197999 81.742001) (end 75.692 79.248) (width 0.508) (layer "B.Cu") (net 27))
 (segment (start 64.262 77.938) (end 62.957999 79.242001) (width 0.508) (layer "B.Cu") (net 27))
 (segment (start 63.636079 81.742001) (end 73.197999 81.742001) (width 0.508) (layer "B.Cu") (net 27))
 (segment (start 69.342 65.278) (end 75.692 71.628) (width 0.508) (layer "F.Cu") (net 24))
 (segment (start 69.342 61.468) (end 69.342 65.278) (width 0.508) (layer "F.Cu") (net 24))
 (segment (start 69.342 58.968) (end 70.89601 60.52201) (width 0.508) (layer "F.Cu") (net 23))
 (segment (start 70.89601 60.52201) (end 70.89601 64.29201) (width 0.508) (layer "F.Cu") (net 23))
 (segment (start 70.89601 64.29201) (end 75.692 69.088) (width 0.508) (layer "F.Cu") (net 23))
 (segment (start 89.662 75.438) (end 90.932 74.168) (width 0.508) (layer "B.Cu") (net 6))
 (segment (start 66.762 75.438) (end 89.662 75.438) (width 0.508) (layer "B.Cu") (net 6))
 (segment (start 75.692 60.783922) (end 75.692 61.468) (width 0.508) (layer "F.Cu") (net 20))
 (segment (start 71.882 56.973922) (end 75.692 60.783922) (width 0.508) (layer "F.Cu") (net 20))
 (segment (start 71.882 52.578) (end 71.882 56.973922) (width 0.508) (layer "F.Cu") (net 20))
 (segment (start 76.962 55.802078) (end 75.692 54.532078) (width 0.508) (layer "F.Cu") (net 17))
 (segment (start 85.852 76.708) (end 76.962 67.818) (width 0.508) (layer "F.Cu") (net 17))
 (segment (start 75.692 54.532078) (end 75.692 53.848) (width 0.508) (layer "F.Cu") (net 17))
 (segment (start 76.962 67.818) (end 76.962 55.802078) (width 0.508) (layer "F.Cu") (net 17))
 (via (at 85.852 76.708) (size 0.8) (drill 0.4) (layers "F.Cu" "B.Cu") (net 17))
 (segment (start 87.376 77.486) (end 87.646 77.486) (width 0.508) (layer "B.Cu") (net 17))
 (segment (start 86.63 77.486) (end 85.852 76.708) (width 0.508) (layer "B.Cu") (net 17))
 (segment (start 87.376 77.486) (end 86.63 77.486) (width 0.508) (layer "B.Cu") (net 17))
 (segment (start 85.614 60.1605) (end 85.5765 60.198) (width 0.508) (layer "B.Cu") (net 34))
 (segment (start 85.614 56.388) (end 85.614 60.1605) (width 0.508) (layer "B.Cu") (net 34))
 (segment (start 85.5765 60.198) (end 83.462 60.198) (width 0.508) (layer "B.Cu") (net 34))
 (segment (start 83.462 60.198) (end 83.142 60.518) (width 0.508) (layer "B.Cu") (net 34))
 (segment (start 81.042 65.593922) (end 81.042 65.278) (width 0.508) (layer "B.Cu") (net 30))
 (segment (start 81.042 62.518) (end 80.942 62.418) (width 0.508) (layer "B.Cu") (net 30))
 (segment (start 76.277922 70.358) (end 81.042 65.593922) (width 0.508) (layer "B.Cu") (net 30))
 (segment (start 81.042 65.278) (end 81.042 62.518) (width 0.508) (layer "B.Cu") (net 30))
 (segment (start 69.342 70.358) (end 76.277922 70.358) (width 0.508) (layer "B.Cu") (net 30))
 (segment (start 87.376 79.486) (end 84.074 79.486) (width 0.508) (layer "B.Cu") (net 36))
 (segment (start 84.074 79.486) (end 80.264 79.486) (width 0.508) (layer "B.Cu") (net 36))
 (segment (start 83.042 65.278) (end 83.09 65.278) (width 0.508) (layer "B.Cu") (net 35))
 (segment (start 83.142 65.178) (end 83.042 65.278) (width 0.508) (layer "B.Cu") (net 35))
 (segment (start 83.142 62.418) (end 83.142 65.178) (width 0.508) (layer "B.Cu") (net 35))
 (segment (start 85.63 65.278) (end 83.042 65.278) (width 0.508) (layer "B.Cu") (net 35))
 (segment (start 79.787999 77.962001) (end 80.264 77.486) (width 0.508) (layer "B.Cu") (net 33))
 (segment (start 66.786001 77.962001) (end 79.787999 77.962001) (width 0.508) (layer "B.Cu") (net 33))
 (segment (start 66.762 77.938) (end 66.786001 77.962001) (width 0.508) (layer "B.Cu") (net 33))
 (segment (start 80.137 77.359) (end 80.264 77.486) (width 0.508) (layer "B.Cu") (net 33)))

